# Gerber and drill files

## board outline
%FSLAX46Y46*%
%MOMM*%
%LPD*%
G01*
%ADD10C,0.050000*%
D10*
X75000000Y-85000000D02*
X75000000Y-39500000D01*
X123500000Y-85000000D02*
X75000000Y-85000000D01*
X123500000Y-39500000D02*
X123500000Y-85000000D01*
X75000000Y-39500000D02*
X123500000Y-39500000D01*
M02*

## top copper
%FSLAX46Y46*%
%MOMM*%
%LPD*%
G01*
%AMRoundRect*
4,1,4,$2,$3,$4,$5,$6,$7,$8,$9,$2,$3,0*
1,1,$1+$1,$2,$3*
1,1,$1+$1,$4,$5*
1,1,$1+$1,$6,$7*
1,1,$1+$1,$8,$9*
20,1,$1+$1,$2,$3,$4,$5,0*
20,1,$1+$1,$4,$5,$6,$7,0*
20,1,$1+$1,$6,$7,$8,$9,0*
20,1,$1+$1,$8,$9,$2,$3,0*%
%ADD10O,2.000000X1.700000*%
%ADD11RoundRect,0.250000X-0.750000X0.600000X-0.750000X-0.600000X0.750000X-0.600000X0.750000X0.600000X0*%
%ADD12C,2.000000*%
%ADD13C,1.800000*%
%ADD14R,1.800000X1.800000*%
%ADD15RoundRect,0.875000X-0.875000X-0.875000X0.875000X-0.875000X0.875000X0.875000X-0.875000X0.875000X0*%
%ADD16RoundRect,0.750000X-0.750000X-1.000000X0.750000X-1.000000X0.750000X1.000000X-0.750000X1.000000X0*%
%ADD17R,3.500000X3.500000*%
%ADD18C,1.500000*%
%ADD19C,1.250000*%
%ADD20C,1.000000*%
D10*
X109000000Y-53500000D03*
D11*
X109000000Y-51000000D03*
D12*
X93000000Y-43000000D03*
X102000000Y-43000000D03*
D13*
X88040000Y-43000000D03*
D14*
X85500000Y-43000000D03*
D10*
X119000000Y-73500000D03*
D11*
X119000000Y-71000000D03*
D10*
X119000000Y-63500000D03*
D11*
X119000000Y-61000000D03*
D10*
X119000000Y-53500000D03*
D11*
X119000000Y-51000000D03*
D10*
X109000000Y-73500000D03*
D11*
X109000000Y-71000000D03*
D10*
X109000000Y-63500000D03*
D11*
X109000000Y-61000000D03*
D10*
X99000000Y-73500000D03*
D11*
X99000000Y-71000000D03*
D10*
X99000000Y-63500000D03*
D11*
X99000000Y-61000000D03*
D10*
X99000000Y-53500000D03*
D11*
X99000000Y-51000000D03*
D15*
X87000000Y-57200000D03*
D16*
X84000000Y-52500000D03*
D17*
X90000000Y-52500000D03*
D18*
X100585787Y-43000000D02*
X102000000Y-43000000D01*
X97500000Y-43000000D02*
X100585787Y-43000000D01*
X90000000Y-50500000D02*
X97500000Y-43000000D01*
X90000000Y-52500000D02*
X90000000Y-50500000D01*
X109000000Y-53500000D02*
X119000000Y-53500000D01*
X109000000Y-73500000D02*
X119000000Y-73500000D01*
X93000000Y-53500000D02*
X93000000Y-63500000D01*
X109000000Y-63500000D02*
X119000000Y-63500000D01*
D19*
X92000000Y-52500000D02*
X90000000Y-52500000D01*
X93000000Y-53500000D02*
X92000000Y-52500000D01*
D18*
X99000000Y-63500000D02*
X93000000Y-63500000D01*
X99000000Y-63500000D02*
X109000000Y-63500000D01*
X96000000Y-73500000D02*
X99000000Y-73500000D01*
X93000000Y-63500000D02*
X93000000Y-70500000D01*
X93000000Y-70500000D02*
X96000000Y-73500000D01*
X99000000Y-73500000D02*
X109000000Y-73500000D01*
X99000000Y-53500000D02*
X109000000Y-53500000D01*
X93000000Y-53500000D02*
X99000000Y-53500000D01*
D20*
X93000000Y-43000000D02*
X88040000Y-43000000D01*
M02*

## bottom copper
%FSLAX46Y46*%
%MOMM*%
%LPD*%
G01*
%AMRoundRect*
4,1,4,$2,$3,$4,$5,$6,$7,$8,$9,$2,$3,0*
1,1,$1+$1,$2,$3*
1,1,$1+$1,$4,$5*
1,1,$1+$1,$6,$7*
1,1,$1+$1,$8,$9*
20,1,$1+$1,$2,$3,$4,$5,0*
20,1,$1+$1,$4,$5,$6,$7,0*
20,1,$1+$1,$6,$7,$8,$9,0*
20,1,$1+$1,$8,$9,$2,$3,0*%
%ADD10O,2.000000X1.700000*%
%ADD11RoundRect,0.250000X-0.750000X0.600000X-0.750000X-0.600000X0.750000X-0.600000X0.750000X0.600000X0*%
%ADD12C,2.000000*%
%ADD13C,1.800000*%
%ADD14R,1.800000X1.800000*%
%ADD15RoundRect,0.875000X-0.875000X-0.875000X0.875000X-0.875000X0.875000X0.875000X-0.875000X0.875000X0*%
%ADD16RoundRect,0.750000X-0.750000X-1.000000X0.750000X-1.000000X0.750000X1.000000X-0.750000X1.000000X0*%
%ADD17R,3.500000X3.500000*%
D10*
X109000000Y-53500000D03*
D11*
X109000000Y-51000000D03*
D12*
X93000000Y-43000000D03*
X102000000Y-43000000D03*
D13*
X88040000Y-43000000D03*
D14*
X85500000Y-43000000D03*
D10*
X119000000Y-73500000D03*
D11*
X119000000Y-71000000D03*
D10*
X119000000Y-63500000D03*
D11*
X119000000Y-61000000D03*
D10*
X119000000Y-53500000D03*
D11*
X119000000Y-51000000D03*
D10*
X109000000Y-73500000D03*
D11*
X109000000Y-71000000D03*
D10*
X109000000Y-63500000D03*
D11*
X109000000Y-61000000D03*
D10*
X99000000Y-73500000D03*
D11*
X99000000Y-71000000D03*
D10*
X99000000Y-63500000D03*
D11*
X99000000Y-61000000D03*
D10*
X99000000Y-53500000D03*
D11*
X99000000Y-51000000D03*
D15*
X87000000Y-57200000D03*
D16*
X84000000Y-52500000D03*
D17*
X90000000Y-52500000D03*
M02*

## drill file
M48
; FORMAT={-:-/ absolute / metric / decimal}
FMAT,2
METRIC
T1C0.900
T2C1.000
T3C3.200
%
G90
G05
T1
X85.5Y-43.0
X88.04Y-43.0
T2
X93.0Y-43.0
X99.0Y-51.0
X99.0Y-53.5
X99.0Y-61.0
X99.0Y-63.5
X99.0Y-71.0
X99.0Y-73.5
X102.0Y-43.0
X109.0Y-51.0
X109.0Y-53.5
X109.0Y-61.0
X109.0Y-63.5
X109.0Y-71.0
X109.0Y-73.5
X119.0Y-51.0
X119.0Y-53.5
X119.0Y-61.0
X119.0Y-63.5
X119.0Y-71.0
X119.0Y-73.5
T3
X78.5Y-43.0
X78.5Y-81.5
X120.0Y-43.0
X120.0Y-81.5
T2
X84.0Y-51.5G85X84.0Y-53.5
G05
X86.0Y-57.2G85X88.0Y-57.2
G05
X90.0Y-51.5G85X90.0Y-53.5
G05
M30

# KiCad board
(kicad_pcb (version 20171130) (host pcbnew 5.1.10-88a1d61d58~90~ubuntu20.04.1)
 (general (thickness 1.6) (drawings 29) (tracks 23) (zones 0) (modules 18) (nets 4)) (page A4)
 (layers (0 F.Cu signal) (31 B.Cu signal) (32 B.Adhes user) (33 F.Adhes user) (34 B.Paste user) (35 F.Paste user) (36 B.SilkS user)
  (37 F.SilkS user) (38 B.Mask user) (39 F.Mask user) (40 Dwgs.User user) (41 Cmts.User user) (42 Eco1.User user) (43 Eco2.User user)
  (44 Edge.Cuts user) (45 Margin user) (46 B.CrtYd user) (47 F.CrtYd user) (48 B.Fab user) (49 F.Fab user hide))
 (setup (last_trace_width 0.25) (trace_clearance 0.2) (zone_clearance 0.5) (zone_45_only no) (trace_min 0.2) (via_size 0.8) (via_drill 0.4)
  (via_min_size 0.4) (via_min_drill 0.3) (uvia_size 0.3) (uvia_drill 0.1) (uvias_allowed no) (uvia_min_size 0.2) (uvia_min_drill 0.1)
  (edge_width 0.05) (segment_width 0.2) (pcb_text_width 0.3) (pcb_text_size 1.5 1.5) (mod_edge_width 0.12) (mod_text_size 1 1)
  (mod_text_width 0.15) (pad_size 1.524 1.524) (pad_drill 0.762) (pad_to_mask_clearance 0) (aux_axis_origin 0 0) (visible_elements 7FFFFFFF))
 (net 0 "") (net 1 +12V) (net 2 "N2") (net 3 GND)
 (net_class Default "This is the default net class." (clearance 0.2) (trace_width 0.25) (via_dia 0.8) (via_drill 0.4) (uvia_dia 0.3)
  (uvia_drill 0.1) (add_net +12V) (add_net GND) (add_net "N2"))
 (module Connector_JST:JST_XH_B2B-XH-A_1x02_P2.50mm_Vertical (layer F.Cu) (at 109 51 270)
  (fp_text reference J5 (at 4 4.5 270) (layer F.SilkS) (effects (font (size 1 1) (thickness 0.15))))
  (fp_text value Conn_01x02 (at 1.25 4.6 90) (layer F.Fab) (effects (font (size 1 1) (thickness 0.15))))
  (pad 2 thru_hole oval (at 2.5 0 270) (size 1.7 2) (drill 1) (layers *.Cu *.Mask) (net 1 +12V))
  (pad 1 thru_hole roundrect (at 0 0 270) (size 1.7 2) (drill 1) (layers *.Cu *.Mask) (roundrect_rratio 0.1470588235294118)))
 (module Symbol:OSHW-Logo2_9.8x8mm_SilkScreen (layer F.Cu) (at 111.5 44)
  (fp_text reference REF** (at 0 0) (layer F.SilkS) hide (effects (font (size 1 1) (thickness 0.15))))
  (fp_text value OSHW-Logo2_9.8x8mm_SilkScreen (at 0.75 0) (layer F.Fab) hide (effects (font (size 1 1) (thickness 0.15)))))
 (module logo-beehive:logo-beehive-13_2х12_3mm (layer F.Cu) (at 88 78)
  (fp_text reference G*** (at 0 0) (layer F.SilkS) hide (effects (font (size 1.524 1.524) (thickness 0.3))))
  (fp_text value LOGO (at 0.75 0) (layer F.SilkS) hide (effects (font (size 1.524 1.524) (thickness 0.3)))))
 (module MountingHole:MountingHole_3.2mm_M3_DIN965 (layer F.Cu) (at 120 81.5)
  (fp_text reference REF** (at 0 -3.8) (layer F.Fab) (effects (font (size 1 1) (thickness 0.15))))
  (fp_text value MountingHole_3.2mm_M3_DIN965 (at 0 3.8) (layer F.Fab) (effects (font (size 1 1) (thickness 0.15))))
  (pad 1 np_thru_hole circle (at 0 0) (size 3.2 3.2) (drill 3.2) (layers *.Cu *.Mask)))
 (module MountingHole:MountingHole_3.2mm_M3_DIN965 (layer F.Cu) (at 78.5 81.5)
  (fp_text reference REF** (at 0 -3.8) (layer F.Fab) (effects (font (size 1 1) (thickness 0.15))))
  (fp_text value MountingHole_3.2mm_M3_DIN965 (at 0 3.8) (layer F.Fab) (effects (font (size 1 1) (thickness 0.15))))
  (pad 1 np_thru_hole circle (at 0 0) (size 3.2 3.2) (drill 3.2) (layers *.Cu *.Mask)))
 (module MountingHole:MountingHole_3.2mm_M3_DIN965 (layer F.Cu) (at 78.5 43)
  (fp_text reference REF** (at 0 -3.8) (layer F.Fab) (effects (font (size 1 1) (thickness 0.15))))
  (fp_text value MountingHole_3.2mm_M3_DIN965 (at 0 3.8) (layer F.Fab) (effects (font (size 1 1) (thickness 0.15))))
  (pad 1 np_thru_hole circle (at 0 0) (size 3.2 3.2) (drill 3.2) (layers *.Cu *.Mask)))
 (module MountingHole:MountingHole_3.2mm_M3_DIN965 (layer F.Cu) (at 120 43)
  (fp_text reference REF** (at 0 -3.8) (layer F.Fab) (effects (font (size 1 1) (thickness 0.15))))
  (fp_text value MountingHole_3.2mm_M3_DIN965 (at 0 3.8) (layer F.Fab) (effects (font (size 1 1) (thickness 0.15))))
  (pad 1 np_thru_hole circle (at 0 0) (size 3.2 3.2) (drill 3.2) (layers *.Cu *.Mask)))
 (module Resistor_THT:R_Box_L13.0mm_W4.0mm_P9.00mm (layer F.Cu) (at 102 43 180)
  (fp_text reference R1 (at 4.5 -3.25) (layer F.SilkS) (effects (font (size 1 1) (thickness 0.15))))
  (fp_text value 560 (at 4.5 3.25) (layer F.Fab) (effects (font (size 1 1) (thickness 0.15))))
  (pad 2 thru_hole circle (at 9 0 180) (size 2 2) (drill 1) (layers *.Cu *.Mask) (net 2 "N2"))
  (pad 1 thru_hole circle (at 0 0 180) (size 2 2) (drill 1) (layers *.Cu *.Mask) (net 1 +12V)))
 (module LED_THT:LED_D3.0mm (layer F.Cu) (at 85.5 43)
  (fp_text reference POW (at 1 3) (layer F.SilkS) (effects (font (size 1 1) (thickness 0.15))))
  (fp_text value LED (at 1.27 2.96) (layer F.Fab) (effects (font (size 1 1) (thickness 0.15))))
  (pad 2 thru_hole circle (at 2.54 0) (size 1.8 1.8) (drill 0.9) (layers *.Cu *.Mask) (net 2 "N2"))
  (pad 1 thru_hole rect (at 0 0) (size 1.8 1.8) (drill 0.9) (layers *.Cu *.Mask)))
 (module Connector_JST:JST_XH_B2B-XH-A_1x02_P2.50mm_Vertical (layer F.Cu) (at 119 71 270)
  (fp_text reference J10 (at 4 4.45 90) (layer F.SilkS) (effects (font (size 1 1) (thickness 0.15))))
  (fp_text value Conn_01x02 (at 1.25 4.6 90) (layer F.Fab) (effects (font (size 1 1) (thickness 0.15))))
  (pad 2 thru_hole oval (at 2.5 0 270) (size 1.7 2) (drill 1) (layers *.Cu *.Mask) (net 1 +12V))
  (pad 1 thru_hole roundrect (at 0 0 270) (size 1.7 2) (drill 1) (layers *.Cu *.Mask) (roundrect_rratio 0.1470588235294118)))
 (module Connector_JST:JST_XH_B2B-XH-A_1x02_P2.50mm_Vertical (layer F.Cu) (at 119 61 270)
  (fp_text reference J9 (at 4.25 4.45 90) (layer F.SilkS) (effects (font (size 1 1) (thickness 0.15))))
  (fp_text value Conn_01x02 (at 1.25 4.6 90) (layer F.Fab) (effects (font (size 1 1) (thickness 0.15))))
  (pad 2 thru_hole oval (at 2.5 0 270) (size 1.7 2) (drill 1) (layers *.Cu *.Mask) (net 1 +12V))
  (pad 1 thru_hole roundrect (at 0 0 270) (size 1.7 2) (drill 1) (layers *.Cu *.Mask) (roundrect_rratio 0.1470588235294118)))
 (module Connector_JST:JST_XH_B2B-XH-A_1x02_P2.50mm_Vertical (layer F.Cu) (at 119 51 270)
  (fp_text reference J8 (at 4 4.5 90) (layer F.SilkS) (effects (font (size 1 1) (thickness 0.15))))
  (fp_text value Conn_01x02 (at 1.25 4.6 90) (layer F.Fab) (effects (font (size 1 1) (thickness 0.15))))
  (pad 2 thru_hole oval (at 2.5 0 270) (size 1.7 2) (drill 1) (layers *.Cu *.Mask) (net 1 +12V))
  (pad 1 thru_hole roundrect (at 0 0 270) (size 1.7 2) (drill 1) (layers *.Cu *.Mask) (roundrect_rratio 0.1470588235294118)))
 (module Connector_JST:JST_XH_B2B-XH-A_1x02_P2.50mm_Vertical (layer F.Cu) (at 109 71 270)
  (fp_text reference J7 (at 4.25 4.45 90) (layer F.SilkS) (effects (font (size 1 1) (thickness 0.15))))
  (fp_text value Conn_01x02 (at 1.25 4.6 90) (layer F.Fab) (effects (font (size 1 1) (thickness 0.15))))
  (pad 2 thru_hole oval (at 2.5 0 270) (size 1.7 2) (drill 1) (layers *.Cu *.Mask) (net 1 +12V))
  (pad 1 thru_hole roundrect (at 0 0 270) (size 1.7 2) (drill 1) (layers *.Cu *.Mask) (roundrect_rratio 0.1470588235294118)))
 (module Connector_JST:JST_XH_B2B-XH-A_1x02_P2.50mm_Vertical (layer F.Cu) (at 109 61 270)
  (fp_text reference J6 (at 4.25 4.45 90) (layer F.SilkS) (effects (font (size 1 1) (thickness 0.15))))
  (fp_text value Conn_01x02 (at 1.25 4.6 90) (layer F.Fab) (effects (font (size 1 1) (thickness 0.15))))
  (pad 2 thru_hole oval (at 2.5 0 270) (size 1.7 2) (drill 1) (layers *.Cu *.Mask) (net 1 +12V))
  (pad 1 thru_hole roundrect (at 0 0 270) (size 1.7 2) (drill 1) (layers *.Cu *.Mask) (roundrect_rratio 0.1470588235294118)))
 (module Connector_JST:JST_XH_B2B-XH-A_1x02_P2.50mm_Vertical (layer F.Cu) (at 99 71 270)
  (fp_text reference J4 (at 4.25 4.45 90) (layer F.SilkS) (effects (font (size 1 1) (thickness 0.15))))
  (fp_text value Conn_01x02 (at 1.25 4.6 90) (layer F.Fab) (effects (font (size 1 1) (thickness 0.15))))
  (pad 2 thru_hole oval (at 2.5 0 270) (size 1.7 2) (drill 1) (layers *.Cu *.Mask) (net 1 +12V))
  (pad 1 thru_hole roundrect (at 0 0 270) (size 1.7 2) (drill 1) (layers *.Cu *.Mask) (roundrect_rratio 0.1470588235294118)))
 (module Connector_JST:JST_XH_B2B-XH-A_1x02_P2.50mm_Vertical (layer F.Cu) (at 99 61 270)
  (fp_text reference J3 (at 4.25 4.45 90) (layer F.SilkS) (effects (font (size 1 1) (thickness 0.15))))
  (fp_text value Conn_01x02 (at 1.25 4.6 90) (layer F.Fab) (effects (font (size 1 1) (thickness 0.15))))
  (pad 2 thru_hole oval (at 2.5 0 270) (size 1.7 2) (drill 1) (layers *.Cu *.Mask) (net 1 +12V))
  (pad 1 thru_hole roundrect (at 0 0 270) (size 1.7 2) (drill 1) (layers *.Cu *.Mask) (roundrect_rratio 0.1470588235294118)))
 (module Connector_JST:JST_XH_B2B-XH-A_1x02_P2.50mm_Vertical (layer F.Cu) (at 99 51 270)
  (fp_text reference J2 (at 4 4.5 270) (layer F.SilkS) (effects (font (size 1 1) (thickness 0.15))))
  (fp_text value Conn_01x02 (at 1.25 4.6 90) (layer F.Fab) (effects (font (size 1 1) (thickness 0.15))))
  (pad 2 thru_hole oval (at 2.5 0 270) (size 1.7 2) (drill 1) (layers *.Cu *.Mask) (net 1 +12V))
  (pad 1 thru_hole roundrect (at 0 0 270) (size 1.7 2) (drill 1) (layers *.Cu *.Mask) (roundrect_rratio 0.1470588235294118)))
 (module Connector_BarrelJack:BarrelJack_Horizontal (layer F.Cu) (at 90 52.5)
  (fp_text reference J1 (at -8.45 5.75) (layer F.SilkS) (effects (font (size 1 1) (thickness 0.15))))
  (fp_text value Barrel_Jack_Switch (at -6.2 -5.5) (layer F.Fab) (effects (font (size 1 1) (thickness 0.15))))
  (pad 3 thru_hole roundrect (at -3 4.7) (size 3.5 3.5) (drill oval 3 1) (layers *.Cu *.Mask) (roundrect_rratio 0.25))
  (pad 2 thru_hole roundrect (at -6 0) (size 3 3.5) (drill oval 1 3) (layers *.Cu *.Mask) (roundrect_rratio 0.25))
  (pad 1 thru_hole rect (at 0 0) (size 3.5 3.5) (drill oval 1 3) (layers *.Cu *.Mask) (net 1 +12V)))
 (gr_line (start 75 85) (end 75 39.5) (layer Edge.Cuts) (width 0.05))
 (gr_line (start 123.5 85) (end 75 85) (layer Edge.Cuts) (width 0.05))
 (gr_line (start 123.5 39.5) (end 123.5 85) (layer Edge.Cuts) (width 0.05))
 (gr_line (start 75 39.5) (end 123.5 39.5) (layer Edge.Cuts) (width 0.05))
 (segment (start 100.585787 43) (end 102 43) (width 1.5) (layer F.Cu) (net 1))
 (segment (start 97.5 43) (end 100.585787 43) (width 1.5) (layer F.Cu) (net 1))
 (segment (start 90 50.5) (end 97.5 43) (width 1.5) (layer F.Cu) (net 1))
 (segment (start 90 52.5) (end 90 50.5) (width 1.5) (layer F.Cu) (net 1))
 (segment (start 109 53.5) (end 119 53.5) (width 1.5) (layer F.Cu) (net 1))
 (segment (start 109 73.5) (end 119 73.5) (width 1.5) (layer F.Cu) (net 1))
 (segment (start 93 53.5) (end 93 63.5) (width 1.5) (layer F.Cu) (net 1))
 (segment (start 109 63.5) (end 119 63.5) (width 1.5) (layer F.Cu) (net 1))
 (segment (start 92 52.5) (end 90 52.5) (width 1.25) (layer F.Cu) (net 1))
 (segment (start 93 53.5) (end 92 52.5) (width 1.25) (layer F.Cu) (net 1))
 (segment (start 99 63.5) (end 93 63.5) (width 1.5) (layer F.Cu) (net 1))
 (segment (start 99 63.5) (end 109 63.5) (width 1.5) (layer F.Cu) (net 1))
 (segment (start 96 73.5) (end 99 73.5) (width 1.5) (layer F.Cu) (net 1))
 (segment (start 93 63.5) (end 93 70.5) (width 1.5) (layer F.Cu) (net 1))
 (segment (start 93 70.5) (end 96 73.5) (width 1.5) (layer F.Cu) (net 1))
 (segment (start 99 73.5) (end 109 73.5) (width 1.5) (layer F.Cu) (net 1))
 (segment (start 99 53.5) (end 109 53.5) (width 1.5) (layer F.Cu) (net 1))
 (segment (start 93 53.5) (end 99 53.5) (width 1.5) (layer F.Cu) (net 1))
 (segment (start 93 43) (end 88.04 43) (width 1) (layer F.Cu) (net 2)))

